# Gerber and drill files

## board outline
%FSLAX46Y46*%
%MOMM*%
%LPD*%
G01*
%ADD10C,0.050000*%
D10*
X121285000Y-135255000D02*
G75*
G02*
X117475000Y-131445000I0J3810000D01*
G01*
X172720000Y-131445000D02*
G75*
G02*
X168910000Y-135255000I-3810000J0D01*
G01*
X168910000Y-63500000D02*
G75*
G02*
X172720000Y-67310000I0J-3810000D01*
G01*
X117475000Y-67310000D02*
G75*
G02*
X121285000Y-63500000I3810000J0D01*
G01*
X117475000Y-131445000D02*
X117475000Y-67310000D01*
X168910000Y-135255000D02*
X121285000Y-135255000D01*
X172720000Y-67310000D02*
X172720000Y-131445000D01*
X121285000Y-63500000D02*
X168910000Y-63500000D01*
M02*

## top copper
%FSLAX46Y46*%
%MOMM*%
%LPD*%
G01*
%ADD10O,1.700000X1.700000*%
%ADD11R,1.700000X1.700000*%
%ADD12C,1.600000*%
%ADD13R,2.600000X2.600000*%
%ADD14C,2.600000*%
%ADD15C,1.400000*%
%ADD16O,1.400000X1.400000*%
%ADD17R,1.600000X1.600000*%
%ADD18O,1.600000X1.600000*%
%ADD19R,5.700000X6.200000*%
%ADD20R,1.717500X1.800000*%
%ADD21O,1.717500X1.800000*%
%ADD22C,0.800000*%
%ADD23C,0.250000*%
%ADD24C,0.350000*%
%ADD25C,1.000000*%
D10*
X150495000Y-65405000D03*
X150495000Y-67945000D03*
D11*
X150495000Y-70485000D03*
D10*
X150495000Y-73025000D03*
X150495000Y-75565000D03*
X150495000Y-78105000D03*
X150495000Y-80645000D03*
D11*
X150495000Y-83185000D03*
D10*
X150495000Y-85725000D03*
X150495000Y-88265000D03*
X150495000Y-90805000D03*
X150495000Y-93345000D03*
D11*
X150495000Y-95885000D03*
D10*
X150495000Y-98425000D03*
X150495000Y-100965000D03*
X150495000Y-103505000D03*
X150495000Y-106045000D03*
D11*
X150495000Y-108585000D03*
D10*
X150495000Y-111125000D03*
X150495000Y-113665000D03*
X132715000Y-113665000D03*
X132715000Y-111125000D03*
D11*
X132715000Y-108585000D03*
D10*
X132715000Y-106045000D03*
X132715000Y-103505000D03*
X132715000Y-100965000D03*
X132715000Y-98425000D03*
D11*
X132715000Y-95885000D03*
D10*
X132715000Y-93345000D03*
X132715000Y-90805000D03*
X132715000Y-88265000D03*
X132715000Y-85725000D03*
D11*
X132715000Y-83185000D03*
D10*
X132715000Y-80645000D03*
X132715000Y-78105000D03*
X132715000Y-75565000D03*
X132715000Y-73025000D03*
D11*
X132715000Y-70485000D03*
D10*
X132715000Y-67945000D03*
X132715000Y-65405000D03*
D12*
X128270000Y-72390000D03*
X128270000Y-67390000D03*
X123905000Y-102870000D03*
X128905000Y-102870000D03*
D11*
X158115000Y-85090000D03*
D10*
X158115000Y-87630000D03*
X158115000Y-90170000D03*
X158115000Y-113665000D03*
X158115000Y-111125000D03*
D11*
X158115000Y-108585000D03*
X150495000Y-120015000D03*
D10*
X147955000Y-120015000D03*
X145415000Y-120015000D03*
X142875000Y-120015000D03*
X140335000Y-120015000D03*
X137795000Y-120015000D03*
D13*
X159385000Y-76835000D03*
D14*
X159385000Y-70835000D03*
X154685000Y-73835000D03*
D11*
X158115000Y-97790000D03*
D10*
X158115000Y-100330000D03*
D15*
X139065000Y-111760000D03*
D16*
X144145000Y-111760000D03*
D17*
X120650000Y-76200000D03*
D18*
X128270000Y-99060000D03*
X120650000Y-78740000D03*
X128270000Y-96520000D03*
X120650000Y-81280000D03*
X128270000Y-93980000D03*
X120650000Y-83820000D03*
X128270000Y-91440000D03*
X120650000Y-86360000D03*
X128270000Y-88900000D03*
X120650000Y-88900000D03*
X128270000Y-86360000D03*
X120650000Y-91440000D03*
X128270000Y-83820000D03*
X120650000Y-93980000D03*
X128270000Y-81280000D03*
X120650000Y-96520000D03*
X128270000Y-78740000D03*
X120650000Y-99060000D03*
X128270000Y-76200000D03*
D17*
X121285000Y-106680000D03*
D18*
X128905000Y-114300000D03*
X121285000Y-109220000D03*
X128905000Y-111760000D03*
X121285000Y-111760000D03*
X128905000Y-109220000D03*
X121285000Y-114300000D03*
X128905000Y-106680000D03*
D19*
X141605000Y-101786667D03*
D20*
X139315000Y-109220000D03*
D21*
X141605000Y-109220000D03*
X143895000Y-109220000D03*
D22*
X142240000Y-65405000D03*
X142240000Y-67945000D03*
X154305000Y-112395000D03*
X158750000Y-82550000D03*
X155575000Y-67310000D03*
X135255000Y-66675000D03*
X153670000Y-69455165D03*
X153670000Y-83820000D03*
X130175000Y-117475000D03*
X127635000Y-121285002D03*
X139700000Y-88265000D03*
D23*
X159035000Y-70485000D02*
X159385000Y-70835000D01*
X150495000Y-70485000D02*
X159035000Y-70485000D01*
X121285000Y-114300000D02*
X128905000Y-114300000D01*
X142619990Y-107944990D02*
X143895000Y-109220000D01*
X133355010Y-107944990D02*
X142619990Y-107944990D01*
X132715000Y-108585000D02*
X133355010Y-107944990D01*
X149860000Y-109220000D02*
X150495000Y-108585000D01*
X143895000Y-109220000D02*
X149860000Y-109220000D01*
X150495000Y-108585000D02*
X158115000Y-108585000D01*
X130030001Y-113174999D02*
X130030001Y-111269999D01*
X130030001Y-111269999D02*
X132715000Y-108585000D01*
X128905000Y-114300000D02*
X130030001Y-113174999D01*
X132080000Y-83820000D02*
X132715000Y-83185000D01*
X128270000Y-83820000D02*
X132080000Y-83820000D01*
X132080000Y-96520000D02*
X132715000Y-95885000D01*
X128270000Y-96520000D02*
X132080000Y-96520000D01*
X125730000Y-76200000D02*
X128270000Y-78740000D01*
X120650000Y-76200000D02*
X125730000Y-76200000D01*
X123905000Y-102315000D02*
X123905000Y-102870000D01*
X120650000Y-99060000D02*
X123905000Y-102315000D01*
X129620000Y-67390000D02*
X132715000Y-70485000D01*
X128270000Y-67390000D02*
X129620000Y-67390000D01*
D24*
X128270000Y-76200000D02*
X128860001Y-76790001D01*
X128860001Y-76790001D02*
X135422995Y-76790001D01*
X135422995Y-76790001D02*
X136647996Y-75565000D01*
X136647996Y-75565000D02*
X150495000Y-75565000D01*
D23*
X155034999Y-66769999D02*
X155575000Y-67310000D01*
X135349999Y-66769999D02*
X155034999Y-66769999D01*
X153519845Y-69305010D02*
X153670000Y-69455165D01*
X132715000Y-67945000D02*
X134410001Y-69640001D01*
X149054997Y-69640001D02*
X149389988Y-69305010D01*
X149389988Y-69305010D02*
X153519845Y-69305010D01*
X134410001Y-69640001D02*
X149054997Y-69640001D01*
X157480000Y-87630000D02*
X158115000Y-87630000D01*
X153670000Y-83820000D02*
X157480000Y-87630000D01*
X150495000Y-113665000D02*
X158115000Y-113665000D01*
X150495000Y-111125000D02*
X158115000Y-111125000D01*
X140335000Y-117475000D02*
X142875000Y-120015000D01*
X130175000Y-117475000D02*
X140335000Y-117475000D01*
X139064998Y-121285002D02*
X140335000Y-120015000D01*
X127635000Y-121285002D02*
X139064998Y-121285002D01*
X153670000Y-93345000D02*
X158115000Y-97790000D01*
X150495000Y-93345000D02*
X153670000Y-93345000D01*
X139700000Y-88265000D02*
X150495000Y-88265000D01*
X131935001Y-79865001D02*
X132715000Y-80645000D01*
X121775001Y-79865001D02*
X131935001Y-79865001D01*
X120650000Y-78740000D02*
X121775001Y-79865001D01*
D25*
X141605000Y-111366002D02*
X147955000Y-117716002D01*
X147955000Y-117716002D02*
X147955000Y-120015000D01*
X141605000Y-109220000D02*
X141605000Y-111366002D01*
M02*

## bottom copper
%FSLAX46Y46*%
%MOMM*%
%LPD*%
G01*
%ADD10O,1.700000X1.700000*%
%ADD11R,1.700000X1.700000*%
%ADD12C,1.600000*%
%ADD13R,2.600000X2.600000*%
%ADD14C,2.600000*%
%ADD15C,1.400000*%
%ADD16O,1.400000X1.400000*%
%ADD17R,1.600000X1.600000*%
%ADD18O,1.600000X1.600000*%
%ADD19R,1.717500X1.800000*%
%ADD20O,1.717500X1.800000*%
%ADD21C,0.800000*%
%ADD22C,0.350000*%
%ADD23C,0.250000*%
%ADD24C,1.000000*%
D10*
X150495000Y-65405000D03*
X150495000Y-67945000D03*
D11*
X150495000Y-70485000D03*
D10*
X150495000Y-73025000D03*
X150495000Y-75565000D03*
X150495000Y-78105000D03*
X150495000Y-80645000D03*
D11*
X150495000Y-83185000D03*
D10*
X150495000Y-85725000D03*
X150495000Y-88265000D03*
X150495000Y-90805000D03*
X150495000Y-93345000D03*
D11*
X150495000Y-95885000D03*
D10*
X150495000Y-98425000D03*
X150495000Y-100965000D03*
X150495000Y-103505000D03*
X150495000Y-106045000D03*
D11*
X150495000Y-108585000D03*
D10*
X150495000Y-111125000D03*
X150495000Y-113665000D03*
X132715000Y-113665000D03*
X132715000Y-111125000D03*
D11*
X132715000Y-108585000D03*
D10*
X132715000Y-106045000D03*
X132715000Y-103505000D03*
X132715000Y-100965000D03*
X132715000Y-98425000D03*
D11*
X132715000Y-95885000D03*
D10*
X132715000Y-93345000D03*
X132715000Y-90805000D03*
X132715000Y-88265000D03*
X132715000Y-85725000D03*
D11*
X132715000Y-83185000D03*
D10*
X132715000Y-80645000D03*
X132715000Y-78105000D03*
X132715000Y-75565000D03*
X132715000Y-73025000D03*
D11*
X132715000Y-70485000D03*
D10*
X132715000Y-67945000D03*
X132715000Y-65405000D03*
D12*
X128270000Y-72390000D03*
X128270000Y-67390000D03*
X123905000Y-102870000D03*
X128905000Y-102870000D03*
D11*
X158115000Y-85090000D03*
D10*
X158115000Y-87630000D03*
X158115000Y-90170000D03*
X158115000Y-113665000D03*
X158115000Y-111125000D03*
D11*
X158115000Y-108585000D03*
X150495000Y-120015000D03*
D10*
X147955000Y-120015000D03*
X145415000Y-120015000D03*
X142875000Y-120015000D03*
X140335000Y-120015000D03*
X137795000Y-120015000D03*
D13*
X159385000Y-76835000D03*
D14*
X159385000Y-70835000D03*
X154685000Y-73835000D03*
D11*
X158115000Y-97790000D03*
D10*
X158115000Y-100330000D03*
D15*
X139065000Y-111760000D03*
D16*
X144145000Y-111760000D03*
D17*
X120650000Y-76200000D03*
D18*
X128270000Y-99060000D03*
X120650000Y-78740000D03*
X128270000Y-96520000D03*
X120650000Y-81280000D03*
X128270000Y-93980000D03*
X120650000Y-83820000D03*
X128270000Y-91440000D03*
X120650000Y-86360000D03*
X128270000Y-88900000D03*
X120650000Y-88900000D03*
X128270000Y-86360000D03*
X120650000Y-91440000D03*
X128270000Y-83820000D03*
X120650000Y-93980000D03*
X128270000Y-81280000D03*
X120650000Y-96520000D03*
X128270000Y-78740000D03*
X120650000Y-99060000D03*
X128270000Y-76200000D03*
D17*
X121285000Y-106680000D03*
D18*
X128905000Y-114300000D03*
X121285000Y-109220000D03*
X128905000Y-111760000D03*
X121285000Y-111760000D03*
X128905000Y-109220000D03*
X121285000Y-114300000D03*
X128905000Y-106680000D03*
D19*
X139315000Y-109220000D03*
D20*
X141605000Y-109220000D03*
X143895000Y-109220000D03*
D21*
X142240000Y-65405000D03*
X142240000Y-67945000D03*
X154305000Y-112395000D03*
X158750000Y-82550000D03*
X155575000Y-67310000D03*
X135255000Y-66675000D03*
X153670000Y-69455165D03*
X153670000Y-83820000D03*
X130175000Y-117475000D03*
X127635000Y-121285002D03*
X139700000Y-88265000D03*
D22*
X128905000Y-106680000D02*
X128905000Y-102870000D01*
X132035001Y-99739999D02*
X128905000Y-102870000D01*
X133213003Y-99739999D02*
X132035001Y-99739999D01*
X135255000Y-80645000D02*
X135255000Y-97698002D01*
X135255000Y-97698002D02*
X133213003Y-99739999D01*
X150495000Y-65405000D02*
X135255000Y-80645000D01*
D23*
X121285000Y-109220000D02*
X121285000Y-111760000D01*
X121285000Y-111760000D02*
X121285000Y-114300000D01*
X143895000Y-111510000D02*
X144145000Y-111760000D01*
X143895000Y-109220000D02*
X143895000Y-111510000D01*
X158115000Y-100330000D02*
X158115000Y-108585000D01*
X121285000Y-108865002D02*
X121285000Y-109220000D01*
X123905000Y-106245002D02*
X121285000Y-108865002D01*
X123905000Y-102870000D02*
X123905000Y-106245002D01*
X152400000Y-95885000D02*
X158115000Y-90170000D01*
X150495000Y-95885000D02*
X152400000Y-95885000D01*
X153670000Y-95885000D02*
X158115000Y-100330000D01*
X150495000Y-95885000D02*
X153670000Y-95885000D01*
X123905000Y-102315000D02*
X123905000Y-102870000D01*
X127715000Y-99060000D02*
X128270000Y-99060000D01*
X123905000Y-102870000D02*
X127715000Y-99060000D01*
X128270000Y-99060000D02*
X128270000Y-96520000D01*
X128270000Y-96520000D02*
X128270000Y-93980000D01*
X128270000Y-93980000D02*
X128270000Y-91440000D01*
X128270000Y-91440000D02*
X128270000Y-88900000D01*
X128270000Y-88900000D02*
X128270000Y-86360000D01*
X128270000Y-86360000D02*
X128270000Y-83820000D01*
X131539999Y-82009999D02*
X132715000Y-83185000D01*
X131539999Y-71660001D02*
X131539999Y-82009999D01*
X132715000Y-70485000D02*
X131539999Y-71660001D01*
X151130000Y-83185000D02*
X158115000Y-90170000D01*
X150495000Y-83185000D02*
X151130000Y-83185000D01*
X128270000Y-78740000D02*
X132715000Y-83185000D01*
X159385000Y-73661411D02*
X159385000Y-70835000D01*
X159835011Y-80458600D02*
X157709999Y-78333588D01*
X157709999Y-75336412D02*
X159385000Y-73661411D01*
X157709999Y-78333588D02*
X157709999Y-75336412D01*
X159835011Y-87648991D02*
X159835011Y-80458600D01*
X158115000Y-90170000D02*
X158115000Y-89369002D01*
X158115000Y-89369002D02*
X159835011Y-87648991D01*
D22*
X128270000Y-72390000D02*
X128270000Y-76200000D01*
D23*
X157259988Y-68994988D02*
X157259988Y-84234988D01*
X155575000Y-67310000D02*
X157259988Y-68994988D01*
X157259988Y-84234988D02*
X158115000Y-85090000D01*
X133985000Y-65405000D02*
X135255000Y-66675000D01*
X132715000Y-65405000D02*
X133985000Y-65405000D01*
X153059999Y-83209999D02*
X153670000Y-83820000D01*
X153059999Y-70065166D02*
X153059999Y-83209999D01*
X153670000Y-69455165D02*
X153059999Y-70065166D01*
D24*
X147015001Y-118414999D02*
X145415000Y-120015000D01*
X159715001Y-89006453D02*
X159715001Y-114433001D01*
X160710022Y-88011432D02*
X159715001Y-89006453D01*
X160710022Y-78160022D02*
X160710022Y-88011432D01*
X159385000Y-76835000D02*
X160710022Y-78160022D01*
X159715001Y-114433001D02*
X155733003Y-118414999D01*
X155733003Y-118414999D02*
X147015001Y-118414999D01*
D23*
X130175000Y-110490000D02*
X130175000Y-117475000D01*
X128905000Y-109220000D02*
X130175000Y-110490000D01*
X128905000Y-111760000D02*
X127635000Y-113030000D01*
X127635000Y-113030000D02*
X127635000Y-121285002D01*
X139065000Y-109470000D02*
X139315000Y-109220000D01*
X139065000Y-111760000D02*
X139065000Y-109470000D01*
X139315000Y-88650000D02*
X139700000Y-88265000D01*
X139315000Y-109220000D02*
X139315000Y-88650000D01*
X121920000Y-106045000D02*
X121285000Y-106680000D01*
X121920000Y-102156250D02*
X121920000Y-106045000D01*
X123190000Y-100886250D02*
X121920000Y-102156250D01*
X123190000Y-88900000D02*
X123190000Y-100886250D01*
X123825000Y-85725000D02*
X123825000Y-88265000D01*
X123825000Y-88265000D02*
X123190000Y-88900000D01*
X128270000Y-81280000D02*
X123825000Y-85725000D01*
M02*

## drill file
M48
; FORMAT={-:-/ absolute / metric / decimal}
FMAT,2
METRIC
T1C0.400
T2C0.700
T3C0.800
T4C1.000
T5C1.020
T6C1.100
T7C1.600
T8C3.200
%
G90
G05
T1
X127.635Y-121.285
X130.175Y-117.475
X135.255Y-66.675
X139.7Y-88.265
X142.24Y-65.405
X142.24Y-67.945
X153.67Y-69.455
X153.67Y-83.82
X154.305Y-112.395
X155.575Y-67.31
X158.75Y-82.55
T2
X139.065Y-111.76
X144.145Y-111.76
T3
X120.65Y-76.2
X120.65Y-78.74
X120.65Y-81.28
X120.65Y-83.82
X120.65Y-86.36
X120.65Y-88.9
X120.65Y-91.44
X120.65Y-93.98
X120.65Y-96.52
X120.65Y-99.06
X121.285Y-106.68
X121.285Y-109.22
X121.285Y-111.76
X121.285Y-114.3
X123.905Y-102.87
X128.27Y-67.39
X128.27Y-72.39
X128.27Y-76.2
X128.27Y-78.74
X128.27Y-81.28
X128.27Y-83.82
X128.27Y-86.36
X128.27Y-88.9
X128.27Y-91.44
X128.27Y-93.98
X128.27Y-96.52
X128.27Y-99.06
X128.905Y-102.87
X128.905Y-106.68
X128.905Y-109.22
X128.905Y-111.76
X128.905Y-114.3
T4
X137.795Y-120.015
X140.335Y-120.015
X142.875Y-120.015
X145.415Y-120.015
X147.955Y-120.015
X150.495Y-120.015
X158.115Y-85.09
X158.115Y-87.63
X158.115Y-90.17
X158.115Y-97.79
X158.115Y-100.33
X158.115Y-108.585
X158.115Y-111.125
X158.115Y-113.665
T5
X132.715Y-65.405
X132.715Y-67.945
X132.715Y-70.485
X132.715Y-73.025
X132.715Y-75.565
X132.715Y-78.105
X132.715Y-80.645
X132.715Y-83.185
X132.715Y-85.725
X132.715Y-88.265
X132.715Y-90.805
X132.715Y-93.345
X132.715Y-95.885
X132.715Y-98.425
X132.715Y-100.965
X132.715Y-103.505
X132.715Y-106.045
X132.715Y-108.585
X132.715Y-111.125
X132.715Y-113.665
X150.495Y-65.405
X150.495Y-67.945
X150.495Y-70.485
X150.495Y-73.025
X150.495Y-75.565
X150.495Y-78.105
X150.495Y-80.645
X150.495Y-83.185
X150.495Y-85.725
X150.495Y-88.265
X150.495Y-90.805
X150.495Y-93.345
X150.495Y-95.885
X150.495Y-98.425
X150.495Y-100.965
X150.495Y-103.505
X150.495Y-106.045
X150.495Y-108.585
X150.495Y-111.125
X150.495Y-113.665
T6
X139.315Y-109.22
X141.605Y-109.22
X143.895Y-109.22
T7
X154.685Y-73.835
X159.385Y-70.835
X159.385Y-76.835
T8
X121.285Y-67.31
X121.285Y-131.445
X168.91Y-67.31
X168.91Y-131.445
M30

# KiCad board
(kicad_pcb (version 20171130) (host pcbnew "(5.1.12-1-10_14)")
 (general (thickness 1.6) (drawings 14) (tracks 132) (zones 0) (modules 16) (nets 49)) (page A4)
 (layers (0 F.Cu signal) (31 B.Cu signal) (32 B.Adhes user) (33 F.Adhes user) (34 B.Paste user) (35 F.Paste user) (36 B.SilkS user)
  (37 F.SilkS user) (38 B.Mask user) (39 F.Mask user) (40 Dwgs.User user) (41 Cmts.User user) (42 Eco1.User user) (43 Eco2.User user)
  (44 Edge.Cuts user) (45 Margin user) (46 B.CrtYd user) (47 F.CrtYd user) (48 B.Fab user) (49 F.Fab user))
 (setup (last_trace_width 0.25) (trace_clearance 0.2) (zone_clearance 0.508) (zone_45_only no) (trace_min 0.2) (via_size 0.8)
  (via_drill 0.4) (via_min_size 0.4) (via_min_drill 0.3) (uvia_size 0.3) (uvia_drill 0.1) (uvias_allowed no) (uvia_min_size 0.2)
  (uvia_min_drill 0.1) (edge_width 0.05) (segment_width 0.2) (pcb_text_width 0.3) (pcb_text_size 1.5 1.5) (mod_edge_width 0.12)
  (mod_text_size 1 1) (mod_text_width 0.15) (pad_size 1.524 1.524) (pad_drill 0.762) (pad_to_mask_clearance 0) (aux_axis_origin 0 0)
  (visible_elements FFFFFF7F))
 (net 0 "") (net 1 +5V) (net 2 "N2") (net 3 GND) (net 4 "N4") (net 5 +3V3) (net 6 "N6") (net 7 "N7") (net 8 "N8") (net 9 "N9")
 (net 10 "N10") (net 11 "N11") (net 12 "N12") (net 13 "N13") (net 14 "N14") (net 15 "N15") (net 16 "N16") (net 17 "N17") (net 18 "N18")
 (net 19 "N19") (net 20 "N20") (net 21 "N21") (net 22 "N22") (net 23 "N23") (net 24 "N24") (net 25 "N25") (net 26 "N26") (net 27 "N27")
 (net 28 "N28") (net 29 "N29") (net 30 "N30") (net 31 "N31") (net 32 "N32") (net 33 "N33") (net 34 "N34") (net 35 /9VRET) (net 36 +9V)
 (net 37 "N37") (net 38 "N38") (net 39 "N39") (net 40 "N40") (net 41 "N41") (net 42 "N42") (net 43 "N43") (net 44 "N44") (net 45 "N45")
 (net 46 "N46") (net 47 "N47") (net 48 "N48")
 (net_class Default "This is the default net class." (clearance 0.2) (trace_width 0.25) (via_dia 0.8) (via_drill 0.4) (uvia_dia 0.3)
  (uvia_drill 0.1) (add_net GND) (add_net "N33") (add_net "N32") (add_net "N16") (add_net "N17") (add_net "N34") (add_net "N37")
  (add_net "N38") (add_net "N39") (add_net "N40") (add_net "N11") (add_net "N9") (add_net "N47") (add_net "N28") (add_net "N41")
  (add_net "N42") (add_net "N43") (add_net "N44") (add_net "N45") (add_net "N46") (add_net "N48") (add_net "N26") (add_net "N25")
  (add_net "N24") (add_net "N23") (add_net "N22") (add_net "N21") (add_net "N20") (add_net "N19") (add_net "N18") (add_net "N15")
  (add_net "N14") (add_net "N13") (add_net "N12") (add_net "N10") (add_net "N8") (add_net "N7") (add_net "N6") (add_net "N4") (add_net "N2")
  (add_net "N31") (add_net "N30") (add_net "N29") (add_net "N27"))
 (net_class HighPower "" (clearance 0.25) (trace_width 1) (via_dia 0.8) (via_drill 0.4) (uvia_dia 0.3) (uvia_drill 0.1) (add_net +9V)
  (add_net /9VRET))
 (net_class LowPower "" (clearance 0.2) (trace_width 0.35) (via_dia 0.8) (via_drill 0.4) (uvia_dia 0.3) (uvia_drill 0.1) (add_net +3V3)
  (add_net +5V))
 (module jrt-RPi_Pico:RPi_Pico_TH (layer F.Cu) (at 141.605 89.535)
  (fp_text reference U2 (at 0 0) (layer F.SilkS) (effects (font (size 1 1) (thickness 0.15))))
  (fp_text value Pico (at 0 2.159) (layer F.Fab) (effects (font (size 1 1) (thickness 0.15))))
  (pad 40 thru_hole oval (at 8.89 -24.13) (size 1.7 1.7) (drill 1.02) (layers *.Cu *.Mask) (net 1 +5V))
  (pad 39 thru_hole oval (at 8.89 -21.59) (size 1.7 1.7) (drill 1.02) (layers *.Cu *.Mask) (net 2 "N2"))
  (pad 38 thru_hole rect (at 8.89 -19.05) (size 1.7 1.7) (drill 1.02) (layers *.Cu *.Mask) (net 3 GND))
  (pad 37 thru_hole oval (at 8.89 -16.51) (size 1.7 1.7) (drill 1.02) (layers *.Cu *.Mask) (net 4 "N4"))
  (pad 36 thru_hole oval (at 8.89 -13.97) (size 1.7 1.7) (drill 1.02) (layers *.Cu *.Mask) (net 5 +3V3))
  (pad 35 thru_hole oval (at 8.89 -11.43) (size 1.7 1.7) (drill 1.02) (layers *.Cu *.Mask) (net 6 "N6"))
  (pad 34 thru_hole oval (at 8.89 -8.89) (size 1.7 1.7) (drill 1.02) (layers *.Cu *.Mask) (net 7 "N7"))
  (pad 33 thru_hole rect (at 8.89 -6.35) (size 1.7 1.7) (drill 1.02) (layers *.Cu *.Mask) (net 3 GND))
  (pad 32 thru_hole oval (at 8.89 -3.81) (size 1.7 1.7) (drill 1.02) (layers *.Cu *.Mask) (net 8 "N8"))
  (pad 31 thru_hole oval (at 8.89 -1.27) (size 1.7 1.7) (drill 1.02) (layers *.Cu *.Mask) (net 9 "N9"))
  (pad 30 thru_hole oval (at 8.89 1.27) (size 1.7 1.7) (drill 1.02) (layers *.Cu *.Mask) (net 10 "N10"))
  (pad 29 thru_hole oval (at 8.89 3.81) (size 1.7 1.7) (drill 1.02) (layers *.Cu *.Mask) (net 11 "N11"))
  (pad 28 thru_hole rect (at 8.89 6.35) (size 1.7 1.7) (drill 1.02) (layers *.Cu *.Mask) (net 3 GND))
  (pad 27 thru_hole oval (at 8.89 8.89) (size 1.7 1.7) (drill 1.02) (layers *.Cu *.Mask) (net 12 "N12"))
  (pad 26 thru_hole oval (at 8.89 11.43) (size 1.7 1.7) (drill 1.02) (layers *.Cu *.Mask) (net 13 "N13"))
  (pad 25 thru_hole oval (at 8.89 13.97) (size 1.7 1.7) (drill 1.02) (layers *.Cu *.Mask) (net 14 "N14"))
  (pad 24 thru_hole oval (at 8.89 16.51) (size 1.7 1.7) (drill 1.02) (layers *.Cu *.Mask) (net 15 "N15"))
  (pad 23 thru_hole rect (at 8.89 19.05) (size 1.7 1.7) (drill 1.02) (layers *.Cu *.Mask) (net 3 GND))
  (pad 22 thru_hole oval (at 8.89 21.59) (size 1.7 1.7) (drill 1.02) (layers *.Cu *.Mask) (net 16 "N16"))
  (pad 21 thru_hole oval (at 8.89 24.13) (size 1.7 1.7) (drill 1.02) (layers *.Cu *.Mask) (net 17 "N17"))
  (pad 20 thru_hole oval (at -8.89 24.13) (size 1.7 1.7) (drill 1.02) (layers *.Cu *.Mask) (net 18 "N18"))
  (pad 19 thru_hole oval (at -8.89 21.59) (size 1.7 1.7) (drill 1.02) (layers *.Cu *.Mask) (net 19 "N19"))
  (pad 18 thru_hole rect (at -8.89 19.05) (size 1.7 1.7) (drill 1.02) (layers *.Cu *.Mask) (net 3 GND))
  (pad 17 thru_hole oval (at -8.89 16.51) (size 1.7 1.7) (drill 1.02) (layers *.Cu *.Mask) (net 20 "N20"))
  (pad 16 thru_hole oval (at -8.89 13.97) (size 1.7 1.7) (drill 1.02) (layers *.Cu *.Mask) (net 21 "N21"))
  (pad 15 thru_hole oval (at -8.89 11.43) (size 1.7 1.7) (drill 1.02) (layers *.Cu *.Mask) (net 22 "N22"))
  (pad 14 thru_hole oval (at -8.89 8.89) (size 1.7 1.7) (drill 1.02) (layers *.Cu *.Mask) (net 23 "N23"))
  (pad 13 thru_hole rect (at -8.89 6.35) (size 1.7 1.7) (drill 1.02) (layers *.Cu *.Mask) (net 3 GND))
  (pad 12 thru_hole oval (at -8.89 3.81) (size 1.7 1.7) (drill 1.02) (layers *.Cu *.Mask) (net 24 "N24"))
  (pad 11 thru_hole oval (at -8.89 1.27) (size 1.7 1.7) (drill 1.02) (layers *.Cu *.Mask) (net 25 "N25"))
  (pad 10 thru_hole oval (at -8.89 -1.27) (size 1.7 1.7) (drill 1.02) (layers *.Cu *.Mask) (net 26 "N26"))
  (pad 9 thru_hole oval (at -8.89 -3.81) (size 1.7 1.7) (drill 1.02) (layers *.Cu *.Mask) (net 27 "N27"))
  (pad 8 thru_hole rect (at -8.89 -6.35) (size 1.7 1.7) (drill 1.02) (layers *.Cu *.Mask) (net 3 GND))
  (pad 7 thru_hole oval (at -8.89 -8.89) (size 1.7 1.7) (drill 1.02) (layers *.Cu *.Mask) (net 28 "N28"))
  (pad 6 thru_hole oval (at -8.89 -11.43) (size 1.7 1.7) (drill 1.02) (layers *.Cu *.Mask) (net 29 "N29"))
  (pad 5 thru_hole oval (at -8.89 -13.97) (size 1.7 1.7) (drill 1.02) (layers *.Cu *.Mask) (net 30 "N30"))
  (pad 4 thru_hole oval (at -8.89 -16.51) (size 1.7 1.7) (drill 1.02) (layers *.Cu *.Mask) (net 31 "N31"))
  (pad 3 thru_hole rect (at -8.89 -19.05) (size 1.7 1.7) (drill 1.02) (layers *.Cu *.Mask) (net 3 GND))
  (pad 2 thru_hole oval (at -8.89 -21.59) (size 1.7 1.7) (drill 1.02) (layers *.Cu *.Mask) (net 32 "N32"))
  (pad 1 thru_hole oval (at -8.89 -24.13) (size 1.7 1.7) (drill 1.02) (layers *.Cu *.Mask) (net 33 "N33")))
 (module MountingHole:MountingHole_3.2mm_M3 (layer F.Cu) (at 168.91 67.31)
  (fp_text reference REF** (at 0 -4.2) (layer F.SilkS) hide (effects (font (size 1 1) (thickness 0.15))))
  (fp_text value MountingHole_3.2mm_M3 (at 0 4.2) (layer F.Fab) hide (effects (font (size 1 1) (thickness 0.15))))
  (pad 1 np_thru_hole circle (at 0 0) (size 3.2 3.2) (drill 3.2) (layers *.Cu *.Mask)))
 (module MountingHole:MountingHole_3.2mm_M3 (layer F.Cu) (at 168.91 131.445)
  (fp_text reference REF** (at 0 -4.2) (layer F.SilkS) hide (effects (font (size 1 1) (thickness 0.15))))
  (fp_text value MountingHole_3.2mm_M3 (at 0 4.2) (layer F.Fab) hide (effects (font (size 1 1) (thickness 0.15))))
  (pad 1 np_thru_hole circle (at 0 0) (size 3.2 3.2) (drill 3.2) (layers *.Cu *.Mask)))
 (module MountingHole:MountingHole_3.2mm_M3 (layer F.Cu) (at 121.285 131.445)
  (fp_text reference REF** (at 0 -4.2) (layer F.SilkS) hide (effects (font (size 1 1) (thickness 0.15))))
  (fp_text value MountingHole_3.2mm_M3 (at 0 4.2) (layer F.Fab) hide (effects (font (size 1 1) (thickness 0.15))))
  (pad 1 np_thru_hole circle (at 0 0) (size 3.2 3.2) (drill 3.2) (layers *.Cu *.Mask)))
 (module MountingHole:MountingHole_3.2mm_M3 (layer F.Cu) (at 121.285 67.31)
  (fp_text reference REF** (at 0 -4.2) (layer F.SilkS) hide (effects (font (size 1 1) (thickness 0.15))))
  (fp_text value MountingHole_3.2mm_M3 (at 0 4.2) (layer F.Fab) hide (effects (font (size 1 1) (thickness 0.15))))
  (pad 1 np_thru_hole circle (at 0 0) (size 3.2 3.2) (drill 3.2) (layers *.Cu *.Mask)))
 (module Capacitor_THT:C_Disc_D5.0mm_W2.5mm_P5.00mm (layer F.Cu) (at 128.27 72.39 90)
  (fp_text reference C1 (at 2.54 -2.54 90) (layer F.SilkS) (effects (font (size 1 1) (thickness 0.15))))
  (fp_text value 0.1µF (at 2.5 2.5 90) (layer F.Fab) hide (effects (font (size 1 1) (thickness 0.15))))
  (pad 1 thru_hole circle (at 0 0 90) (size 1.6 1.6) (drill 0.8) (layers *.Cu *.Mask) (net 5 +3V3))
  (pad 2 thru_hole circle (at 5 0 90) (size 1.6 1.6) (drill 0.8) (layers *.Cu *.Mask) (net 3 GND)))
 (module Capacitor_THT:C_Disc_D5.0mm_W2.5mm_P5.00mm (layer F.Cu) (at 128.905 102.87 180)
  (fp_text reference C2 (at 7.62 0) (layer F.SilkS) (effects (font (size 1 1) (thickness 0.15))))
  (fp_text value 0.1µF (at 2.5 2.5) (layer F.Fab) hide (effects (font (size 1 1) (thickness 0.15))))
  (pad 2 thru_hole circle (at 5 0 180) (size 1.6 1.6) (drill 0.8) (layers *.Cu *.Mask) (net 3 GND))
  (pad 1 thru_hole circle (at 0 0 180) (size 1.6 1.6) (drill 0.8) (layers *.Cu *.Mask) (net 1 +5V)))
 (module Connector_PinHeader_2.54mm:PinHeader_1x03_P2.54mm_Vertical (layer F.Cu) (at 158.115 85.09)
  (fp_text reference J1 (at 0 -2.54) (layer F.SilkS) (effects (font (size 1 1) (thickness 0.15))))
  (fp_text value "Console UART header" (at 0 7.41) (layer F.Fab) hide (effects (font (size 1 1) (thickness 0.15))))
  (pad 1 thru_hole rect (at 0 0) (size 1.7 1.7) (drill 1) (layers *.Cu *.Mask) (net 33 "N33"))
  (pad 2 thru_hole oval (at 0 2.54) (size 1.7 1.7) (drill 1) (layers *.Cu *.Mask) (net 32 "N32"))
  (pad 3 thru_hole oval (at 0 5.08) (size 1.7 1.7) (drill 1) (layers *.Cu *.Mask) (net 3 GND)))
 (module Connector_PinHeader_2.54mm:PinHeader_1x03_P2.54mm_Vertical (layer F.Cu) (at 158.115 108.585)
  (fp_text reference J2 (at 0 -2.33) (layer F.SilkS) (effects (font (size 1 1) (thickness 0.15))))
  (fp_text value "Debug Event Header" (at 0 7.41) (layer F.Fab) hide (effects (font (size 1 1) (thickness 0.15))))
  (pad 3 thru_hole oval (at 0 5.08) (size 1.7 1.7) (drill 1) (layers *.Cu *.Mask) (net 17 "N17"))
  (pad 2 thru_hole oval (at 0 2.54) (size 1.7 1.7) (drill 1) (layers *.Cu *.Mask) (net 16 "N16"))
  (pad 1 thru_hole rect (at 0 0) (size 1.7 1.7) (drill 1) (layers *.Cu *.Mask) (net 3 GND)))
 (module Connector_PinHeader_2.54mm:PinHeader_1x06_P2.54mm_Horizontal (layer F.Cu) (at 150.495 120.015 270)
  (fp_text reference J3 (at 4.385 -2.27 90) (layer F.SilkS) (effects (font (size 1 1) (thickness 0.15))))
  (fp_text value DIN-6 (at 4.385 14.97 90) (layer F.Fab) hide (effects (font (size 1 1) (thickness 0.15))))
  (pad 1 thru_hole rect (at 0 0 270) (size 1.7 1.7) (drill 1) (layers *.Cu *.Mask) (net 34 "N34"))
  (pad 2 thru_hole oval (at 0 2.54 270) (size 1.7 1.7) (drill 1) (layers *.Cu *.Mask) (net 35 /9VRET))
  (pad 3 thru_hole oval (at 0 5.08 270) (size 1.7 1.7) (drill 1) (layers *.Cu *.Mask) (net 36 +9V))
  (pad 4 thru_hole oval (at 0 7.62 270) (size 1.7 1.7) (drill 1) (layers *.Cu *.Mask) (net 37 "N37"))
  (pad 5 thru_hole oval (at 0 10.16 270) (size 1.7 1.7) (drill 1) (layers *.Cu *.Mask) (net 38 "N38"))
  (pad 6 thru_hole oval (at 0 12.7 270) (size 1.7 1.7) (drill 1) (layers *.Cu *.Mask) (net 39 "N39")))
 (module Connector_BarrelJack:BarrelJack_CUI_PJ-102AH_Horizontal (layer F.Cu) (at 159.385 76.835 180)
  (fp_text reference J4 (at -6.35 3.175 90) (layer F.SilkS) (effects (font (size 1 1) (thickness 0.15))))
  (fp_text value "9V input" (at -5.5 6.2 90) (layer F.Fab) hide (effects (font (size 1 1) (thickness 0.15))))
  (pad 1 thru_hole rect (at 0 0 180) (size 2.6 2.6) (drill 1.6) (layers *.Cu *.Mask) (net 36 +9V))
  (pad 2 thru_hole circle (at 0 6 180) (size 2.6 2.6) (drill 1.6) (layers *.Cu *.Mask) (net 3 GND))
  (pad 3 thru_hole circle (at 4.7 3 180) (size 2.6 2.6) (drill 1.6) (layers *.Cu *.Mask) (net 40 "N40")))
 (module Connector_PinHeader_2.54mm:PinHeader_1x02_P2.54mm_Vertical (layer F.Cu) (at 158.115 97.79)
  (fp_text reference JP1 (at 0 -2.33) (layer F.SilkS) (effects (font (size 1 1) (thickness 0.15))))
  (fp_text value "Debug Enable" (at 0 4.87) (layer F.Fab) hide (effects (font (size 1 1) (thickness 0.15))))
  (pad 1 thru_hole rect (at 0 0) (size 1.7 1.7) (drill 1) (layers *.Cu *.Mask) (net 11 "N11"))
  (pad 2 thru_hole oval (at 0 2.54) (size 1.7 1.7) (drill 1) (layers *.Cu *.Mask) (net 3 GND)))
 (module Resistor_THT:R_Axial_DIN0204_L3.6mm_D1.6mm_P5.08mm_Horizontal (layer F.Cu) (at 139.065 111.76)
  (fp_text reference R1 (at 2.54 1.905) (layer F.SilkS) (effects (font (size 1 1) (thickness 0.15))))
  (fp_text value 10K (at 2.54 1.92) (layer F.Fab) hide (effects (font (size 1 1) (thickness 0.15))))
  (pad 1 thru_hole circle (at 0 0) (size 1.4 1.4) (drill 0.7) (layers *.Cu *.Mask) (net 9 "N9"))
  (pad 2 thru_hole oval (at 5.08 0) (size 1.4 1.4) (drill 0.7) (layers *.Cu *.Mask) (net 3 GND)))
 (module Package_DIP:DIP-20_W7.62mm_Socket (layer F.Cu) (at 120.65 76.2)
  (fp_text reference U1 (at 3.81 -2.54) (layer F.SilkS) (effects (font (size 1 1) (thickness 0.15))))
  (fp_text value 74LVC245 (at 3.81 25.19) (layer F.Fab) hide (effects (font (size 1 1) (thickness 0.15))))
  (pad 1 thru_hole rect (at 0 0) (size 1.6 1.6) (drill 0.8) (layers *.Cu *.Mask) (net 3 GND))
  (pad 11 thru_hole oval (at 7.62 22.86) (size 1.6 1.6) (drill 0.8) (layers *.Cu *.Mask) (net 3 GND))
  (pad 2 thru_hole oval (at 0 2.54) (size 1.6 1.6) (drill 0.8) (layers *.Cu *.Mask) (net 28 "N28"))
  (pad 12 thru_hole oval (at 7.62 20.32) (size 1.6 1.6) (drill 0.8) (layers *.Cu *.Mask) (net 3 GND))
  (pad 3 thru_hole oval (at 0 5.08) (size 1.6 1.6) (drill 0.8) (layers *.Cu *.Mask) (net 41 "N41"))
  (pad 13 thru_hole oval (at 7.62 17.78) (size 1.6 1.6) (drill 0.8) (layers *.Cu *.Mask) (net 3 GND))
  (pad 4 thru_hole oval (at 0 7.62) (size 1.6 1.6) (drill 0.8) (layers *.Cu *.Mask) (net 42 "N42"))
  (pad 14 thru_hole oval (at 7.62 15.24) (size 1.6 1.6) (drill 0.8) (layers *.Cu *.Mask) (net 3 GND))
  (pad 5 thru_hole oval (at 0 10.16) (size 1.6 1.6) (drill 0.8) (layers *.Cu *.Mask) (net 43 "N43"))
  (pad 15 thru_hole oval (at 7.62 12.7) (size 1.6 1.6) (drill 0.8) (layers *.Cu *.Mask) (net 3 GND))
  (pad 6 thru_hole oval (at 0 12.7) (size 1.6 1.6) (drill 0.8) (layers *.Cu *.Mask) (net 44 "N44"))
  (pad 16 thru_hole oval (at 7.62 10.16) (size 1.6 1.6) (drill 0.8) (layers *.Cu *.Mask) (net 3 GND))
  (pad 7 thru_hole oval (at 0 15.24) (size 1.6 1.6) (drill 0.8) (layers *.Cu *.Mask) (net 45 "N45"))
  (pad 17 thru_hole oval (at 7.62 7.62) (size 1.6 1.6) (drill 0.8) (layers *.Cu *.Mask) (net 3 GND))
  (pad 8 thru_hole oval (at 0 17.78) (size 1.6 1.6) (drill 0.8) (layers *.Cu *.Mask) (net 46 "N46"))
  (pad 18 thru_hole oval (at 7.62 5.08) (size 1.6 1.6) (drill 0.8) (layers *.Cu *.Mask) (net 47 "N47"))
  (pad 9 thru_hole oval (at 0 20.32) (size 1.6 1.6) (drill 0.8) (layers *.Cu *.Mask) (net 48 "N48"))
  (pad 19 thru_hole oval (at 7.62 2.54) (size 1.6 1.6) (drill 0.8) (layers *.Cu *.Mask) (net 3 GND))
  (pad 10 thru_hole oval (at 0 22.86) (size 1.6 1.6) (drill 0.8) (layers *.Cu *.Mask) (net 3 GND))
  (pad 20 thru_hole oval (at 7.62 0) (size 1.6 1.6) (drill 0.8) (layers *.Cu *.Mask) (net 5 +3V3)))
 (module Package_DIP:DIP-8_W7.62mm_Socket (layer F.Cu) (at 121.285 106.68)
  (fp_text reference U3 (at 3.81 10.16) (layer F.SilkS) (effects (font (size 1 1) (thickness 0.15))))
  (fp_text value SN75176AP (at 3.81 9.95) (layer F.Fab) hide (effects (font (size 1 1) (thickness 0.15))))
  (pad 1 thru_hole rect (at 0 0) (size 1.6 1.6) (drill 0.8) (layers *.Cu *.Mask) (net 47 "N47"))
  (pad 5 thru_hole oval (at 7.62 7.62) (size 1.6 1.6) (drill 0.8) (layers *.Cu *.Mask) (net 3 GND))
  (pad 2 thru_hole oval (at 0 2.54) (size 1.6 1.6) (drill 0.8) (layers *.Cu *.Mask) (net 3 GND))
  (pad 6 thru_hole oval (at 7.62 5.08) (size 1.6 1.6) (drill 0.8) (layers *.Cu *.Mask) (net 38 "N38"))
  (pad 3 thru_hole oval (at 0 5.08) (size 1.6 1.6) (drill 0.8) (layers *.Cu *.Mask) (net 3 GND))
  (pad 7 thru_hole oval (at 7.62 2.54) (size 1.6 1.6) (drill 0.8) (layers *.Cu *.Mask) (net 37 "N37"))
  (pad 4 thru_hole oval (at 0 7.62) (size 1.6 1.6) (drill 0.8) (layers *.Cu *.Mask) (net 3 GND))
  (pad 8 thru_hole oval (at 7.62 0) (size 1.6 1.6) (drill 0.8) (layers *.Cu *.Mask) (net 1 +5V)))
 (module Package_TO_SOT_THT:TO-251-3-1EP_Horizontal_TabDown (layer F.Cu) (at 139.315 109.22)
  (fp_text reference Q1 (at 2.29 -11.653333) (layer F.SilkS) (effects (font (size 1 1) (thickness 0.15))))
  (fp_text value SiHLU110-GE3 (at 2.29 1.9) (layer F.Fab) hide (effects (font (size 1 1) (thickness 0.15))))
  (pad 4 smd rect (at 2.29 -7.433333) (size 5.7 6.2) (layers F.Cu F.Paste F.Mask))
  (pad 1 thru_hole rect (at 0 0) (size 1.7175 1.8) (drill 1.1) (layers *.Cu *.Mask) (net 9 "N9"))
  (pad 2 thru_hole oval (at 2.29 0) (size 1.7175 1.8) (drill 1.1) (layers *.Cu *.Mask) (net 35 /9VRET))
  (pad 3 thru_hole oval (at 4.58 0) (size 1.7175 1.8) (drill 1.1) (layers *.Cu *.Mask) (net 3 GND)))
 (gr_arc (start 121.285 131.445) (end 117.475 131.445) (angle -90) (layer Edge.Cuts) (width 0.05))
 (gr_arc (start 168.91 131.445) (end 168.91 135.255) (angle -90) (layer Edge.Cuts) (width 0.05))
 (gr_arc (start 168.91 67.31) (end 172.72 67.31) (angle -90) (layer Edge.Cuts) (width 0.05))
 (gr_arc (start 121.285 67.31) (end 121.285 63.5) (angle -90) (layer Edge.Cuts) (width 0.05))
 (gr_line (start 117.475 131.445) (end 117.475 67.31) (layer Edge.Cuts) (width 0.05))
 (gr_line (start 168.91 135.255) (end 121.285 135.255) (layer Edge.Cuts) (width 0.05))
 (gr_line (start 172.72 67.31) (end 172.72 131.445) (layer Edge.Cuts) (width 0.05))
 (gr_line (start 121.285 63.5) (end 168.91 63.5) (layer Edge.Cuts) (width 0.05))
 (segment (start 128.905 106.68) (end 128.905 102.87) (width 0.35) (layer B.Cu) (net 1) (status 30))
 (segment (start 132.035001 99.739999) (end 128.905 102.87) (width 0.35) (layer B.Cu) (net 1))
 (segment (start 133.213003 99.739999) (end 132.035001 99.739999) (width 0.35) (layer B.Cu) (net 1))
 (segment (start 135.255 80.645) (end 135.255 97.698002) (width 0.35) (layer B.Cu) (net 1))
 (segment (start 135.255 97.698002) (end 133.213003 99.739999) (width 0.35) (layer B.Cu) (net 1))
 (segment (start 150.495 65.405) (end 135.255 80.645) (width 0.35) (layer B.Cu) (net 1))
 (segment (start 159.035 70.485) (end 159.385 70.835) (width 0.25) (layer F.Cu) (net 3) (status 30))
 (segment (start 150.495 70.485) (end 159.035 70.485) (width 0.25) (layer F.Cu) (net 3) (status 30))
 (segment (start 121.285 109.22) (end 121.285 111.76) (width 0.25) (layer B.Cu) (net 3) (status 30))
 (segment (start 121.285 111.76) (end 121.285 114.3) (width 0.25) (layer B.Cu) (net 3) (status 30))
 (segment (start 121.285 114.3) (end 128.905 114.3) (width 0.25) (layer F.Cu) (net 3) (status 30))
 (segment (start 142.61999 107.94499) (end 143.895 109.22) (width 0.25) (layer F.Cu) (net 3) (status 20))
 (segment (start 133.35501 107.94499) (end 142.61999 107.94499) (width 0.25) (layer F.Cu) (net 3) (status 10))
 (segment (start 132.715 108.585) (end 133.35501 107.94499) (width 0.25) (layer F.Cu) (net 3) (status 30))
 (segment (start 143.895 111.51) (end 144.145 111.76) (width 0.25) (layer B.Cu) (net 3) (status 30))
 (segment (start 143.895 109.22) (end 143.895 111.51) (width 0.25) (layer B.Cu) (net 3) (status 30))
 (segment (start 149.86 109.22) (end 150.495 108.585) (width 0.25) (layer F.Cu) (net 3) (status 30))
 (segment (start 143.895 109.22) (end 149.86 109.22) (width 0.25) (layer F.Cu) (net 3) (status 30))
 (segment (start 150.495 108.585) (end 158.115 108.585) (width 0.25) (layer F.Cu) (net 3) (status 30))
 (segment (start 158.115 100.33) (end 158.115 108.585) (width 0.25) (layer B.Cu) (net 3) (status 30))
 (segment (start 121.285 108.865002) (end 121.285 109.22) (width 0.25) (layer B.Cu) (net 3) (status 30))
 (segment (start 123.905 106.245002) (end 121.285 108.865002) (width 0.25) (layer B.Cu) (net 3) (status 20))
 (segment (start 123.905 102.87) (end 123.905 106.245002) (width 0.25) (layer B.Cu) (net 3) (status 10))
 (segment (start 130.030001 113.174999) (end 130.030001 111.269999) (width 0.25) (layer F.Cu) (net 3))
 (segment (start 130.030001 111.269999) (end 132.715 108.585) (width 0.25) (layer F.Cu) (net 3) (status 20))
 (segment (start 128.905 114.3) (end 130.030001 113.174999) (width 0.25) (layer F.Cu) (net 3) (status 10))
 (segment (start 152.4 95.885) (end 158.115 90.17) (width 0.25) (layer B.Cu) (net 3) (status 20))
 (segment (start 150.495 95.885) (end 152.4 95.885) (width 0.25) (layer B.Cu) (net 3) (status 10))
 (segment (start 153.67 95.885) (end 158.115 100.33) (width 0.25) (layer B.Cu) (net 3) (status 20))
 (segment (start 150.495 95.885) (end 153.67 95.885) (width 0.25) (layer B.Cu) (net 3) (status 10))
 (segment (start 123.905 102.315) (end 123.905 102.87) (width 0.25) (layer B.Cu) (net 3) (status 30))
 (segment (start 127.715 99.06) (end 128.27 99.06) (width 0.25) (layer B.Cu) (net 3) (status 30))
 (segment (start 123.905 102.87) (end 127.715 99.06) (width 0.25) (layer B.Cu) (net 3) (status 30))
 (segment (start 128.27 99.06) (end 128.27 96.52) (width 0.25) (layer B.Cu) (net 3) (status 30))
 (segment (start 128.27 96.52) (end 128.27 93.98) (width 0.25) (layer B.Cu) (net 3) (status 30))
 (segment (start 128.27 93.98) (end 128.27 91.44) (width 0.25) (layer B.Cu) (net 3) (status 30))
 (segment (start 128.27 91.44) (end 128.27 88.9) (width 0.25) (layer B.Cu) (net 3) (status 30))
 (segment (start 128.27 88.9) (end 128.27 86.36) (width 0.25) (layer B.Cu) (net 3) (status 30))
 (segment (start 128.27 86.36) (end 128.27 83.82) (width 0.25) (layer B.Cu) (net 3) (status 30))
 (segment (start 132.08 83.82) (end 132.715 83.185) (width 0.25) (layer F.Cu) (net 3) (status 30))
 (segment (start 128.27 83.82) (end 132.08 83.82) (width 0.25) (layer F.Cu) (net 3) (status 30))
 (segment (start 132.08 96.52) (end 132.715 95.885) (width 0.25) (layer F.Cu) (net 3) (status 30))
 (segment (start 128.27 96.52) (end 132.08 96.52) (width 0.25) (layer F.Cu) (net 3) (status 30))
 (segment (start 125.73 76.2) (end 128.27 78.74) (width 0.25) (layer F.Cu) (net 3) (status 20))
 (segment (start 120.65 76.2) (end 125.73 76.2) (width 0.25) (layer F.Cu) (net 3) (status 10))
 (segment (start 123.905 102.315) (end 123.905 102.87) (width 0.25) (layer F.Cu) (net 3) (status 30))
 (segment (start 120.65 99.06) (end 123.905 102.315) (width 0.25) (layer F.Cu) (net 3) (status 30))
 (segment (start 129.62 67.39) (end 132.715 70.485) (width 0.25) (layer F.Cu) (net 3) (status 20))
 (segment (start 128.27 67.39) (end 129.62 67.39) (width 0.25) (layer F.Cu) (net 3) (status 10))
 (segment (start 131.539999 82.009999) (end 132.715 83.185) (width 0.25) (layer B.Cu) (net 3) (status 20))
 (segment (start 131.539999 71.660001) (end 131.539999 82.009999) (width 0.25) (layer B.Cu) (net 3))
 (segment (start 132.715 70.485) (end 131.539999 71.660001) (width 0.25) (layer B.Cu) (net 3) (status 10))
 (segment (start 151.13 83.185) (end 158.115 90.17) (width 0.25) (layer B.Cu) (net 3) (status 30))
 (segment (start 150.495 83.185) (end 151.13 83.185) (width 0.25) (layer B.Cu) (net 3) (status 30))
 (segment (start 128.27 78.74) (end 132.715 83.185) (width 0.25) (layer B.Cu) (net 3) (status 30))
 (segment (start 159.385 73.661411) (end 159.385 70.835) (width 0.25) (layer B.Cu) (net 3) (status 20))
 (segment (start 159.835011 80.4586) (end 157.709999 78.333588) (width 0.25) (layer B.Cu) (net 3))
 (segment (start 157.709999 75.336412) (end 159.385 73.661411) (width 0.25) (layer B.Cu) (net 3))
 (segment (start 157.709999 78.333588) (end 157.709999 75.336412) (width 0.25) (layer B.Cu) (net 3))
 (segment (start 159.835011 87.648991) (end 159.835011 80.4586) (width 0.25) (layer B.Cu) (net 3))
 (segment (start 158.115 90.17) (end 158.115 89.369002) (width 0.25) (layer B.Cu) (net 3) (status 30))
 (segment (start 158.115 89.369002) (end 159.835011 87.648991) (width 0.25) (layer B.Cu) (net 3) (status 10))
 (via (at 142.24 65.405) (size 0.8) (drill 0.4) (layers F.Cu B.Cu) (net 3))
 (via (at 142.24 67.945) (size 0.8) (drill 0.4) (layers F.Cu B.Cu) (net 3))
 (via (at 154.305 112.395) (size 0.8) (drill 0.4) (layers F.Cu B.Cu) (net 3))
 (via (at 158.75 82.55) (size 0.8) (drill 0.4) (layers F.Cu B.Cu) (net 3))
 (segment (start 128.27 72.39) (end 128.27 76.2) (width 0.35) (layer B.Cu) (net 5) (status 30))
 (segment (start 128.27 76.2) (end 128.860001 76.790001) (width 0.35) (layer F.Cu) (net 5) (status 10))
 (segment (start 128.860001 76.790001) (end 135.422995 76.790001) (width 0.35) (layer F.Cu) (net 5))
 (segment (start 135.422995 76.790001) (end 136.647996 75.565) (width 0.35) (layer F.Cu) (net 5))
 (segment (start 136.647996 75.565) (end 150.495 75.565) (width 0.35) (layer F.Cu) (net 5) (status 20))
 (via (at 155.575 67.31) (size 0.8) (drill 0.4) (layers F.Cu B.Cu) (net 33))
 (segment (start 155.034999 66.769999) (end 155.575 67.31) (width 0.25) (layer F.Cu) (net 33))
 (segment (start 135.349999 66.769999) (end 155.034999 66.769999) (width 0.25) (layer F.Cu) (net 33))
 (segment (start 157.259988 68.994988) (end 157.259988 84.234988) (width 0.25) (layer B.Cu) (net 33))
 (segment (start 155.575 67.31) (end 157.259988 68.994988) (width 0.25) (layer B.Cu) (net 33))
 (segment (start 157.259988 84.234988) (end 158.115 85.09) (width 0.25) (layer B.Cu) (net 33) (status 20))
 (segment (start 133.985 65.405) (end 135.255 66.675) (width 0.25) (layer B.Cu) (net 33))
 (via (at 135.255 66.675) (size 0.8) (drill 0.4) (layers F.Cu B.Cu) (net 33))
 (segment (start 132.715 65.405) (end 133.985 65.405) (width 0.25) (layer B.Cu) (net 33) (status 10))
 (segment (start 153.519845 69.30501) (end 153.67 69.455165) (width 0.25) (layer F.Cu) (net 32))
 (segment (start 132.715 67.945) (end 134.410001 69.640001) (width 0.25) (layer F.Cu) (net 32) (status 10))
 (segment (start 149.054997 69.640001) (end 149.389988 69.30501) (width 0.25) (layer F.Cu) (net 32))
 (segment (start 149.389988 69.30501) (end 153.519845 69.30501) (width 0.25) (layer F.Cu) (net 32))
 (segment (start 134.410001 69.640001) (end 149.054997 69.640001) (width 0.25) (layer F.Cu) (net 32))
 (via (at 153.67 69.455165) (size 0.8) (drill 0.4) (layers F.Cu B.Cu) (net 32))
 (via (at 153.67 83.82) (size 0.8) (drill 0.4) (layers F.Cu B.Cu) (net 32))
 (segment (start 153.059999 83.209999) (end 153.67 83.82) (width 0.25) (layer B.Cu) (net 32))
 (segment (start 153.059999 70.065166) (end 153.059999 83.209999) (width 0.25) (layer B.Cu) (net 32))
 (segment (start 153.67 69.455165) (end 153.059999 70.065166) (width 0.25) (layer B.Cu) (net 32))
 (segment (start 157.48 87.63) (end 158.115 87.63) (width 0.25) (layer F.Cu) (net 32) (status 30))
 (segment (start 153.67 83.82) (end 157.48 87.63) (width 0.25) (layer F.Cu) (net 32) (status 20))
 (segment (start 150.495 113.665) (end 158.115 113.665) (width 0.25) (layer F.Cu) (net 17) (status 30))
 (segment (start 150.495 111.125) (end 158.115 111.125) (width 0.25) (layer F.Cu) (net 16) (status 30))
 (segment (start 147.015001 118.414999) (end 145.415 120.015) (width 1) (layer B.Cu) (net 36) (status 20))
 (segment (start 159.715001 89.006453) (end 159.715001 114.433001) (width 1) (layer B.Cu) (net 36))
 (segment (start 160.710022 88.011432) (end 159.715001 89.006453) (width 1) (layer B.Cu) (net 36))
 (segment (start 160.710022 78.160022) (end 160.710022 88.011432) (width 1) (layer B.Cu) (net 36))
 (segment (start 159.385 76.835) (end 160.710022 78.160022) (width 1) (layer B.Cu) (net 36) (status 10))
 (segment (start 159.715001 114.433001) (end 155.733003 118.414999) (width 1) (layer B.Cu) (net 36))
 (segment (start 155.733003 118.414999) (end 147.015001 118.414999) (width 1) (layer B.Cu) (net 36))
 (via (at 130.175 117.475) (size 0.8) (drill 0.4) (layers F.Cu B.Cu) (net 37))
 (segment (start 130.175 110.49) (end 130.175 117.475) (width 0.25) (layer B.Cu) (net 37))
 (segment (start 128.905 109.22) (end 130.175 110.49) (width 0.25) (layer B.Cu) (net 37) (status 10))
 (segment (start 140.335 117.475) (end 142.875 120.015) (width 0.25) (layer F.Cu) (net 37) (status 20))
 (segment (start 130.175 117.475) (end 140.335 117.475) (width 0.25) (layer F.Cu) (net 37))
 (via (at 127.635 121.285002) (size 0.8) (drill 0.4) (layers F.Cu B.Cu) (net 38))
 (segment (start 128.905 111.76) (end 127.635 113.03) (width 0.25) (layer B.Cu) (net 38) (status 10))
 (segment (start 127.635 113.03) (end 127.635 121.285002) (width 0.25) (layer B.Cu) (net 38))
 (segment (start 139.064998 121.285002) (end 140.335 120.015) (width 0.25) (layer F.Cu) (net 38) (status 20))
 (segment (start 127.635 121.285002) (end 139.064998 121.285002) (width 0.25) (layer F.Cu) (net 38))
 (segment (start 153.67 93.345) (end 158.115 97.79) (width 0.25) (layer F.Cu) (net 11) (status 20))
 (segment (start 150.495 93.345) (end 153.67 93.345) (width 0.25) (layer F.Cu) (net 11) (status 10))
 (segment (start 139.065 109.47) (end 139.315 109.22) (width 0.25) (layer B.Cu) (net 9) (status 30))
 (segment (start 139.065 111.76) (end 139.065 109.47) (width 0.25) (layer B.Cu) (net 9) (status 30))
 (via (at 139.7 88.265) (size 0.8) (drill 0.4) (layers F.Cu B.Cu) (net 9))
 (segment (start 139.315 88.65) (end 139.7 88.265) (width 0.25) (layer B.Cu) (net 9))
 (segment (start 139.315 109.22) (end 139.315 88.65) (width 0.25) (layer B.Cu) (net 9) (status 10))
 (segment (start 139.7 88.265) (end 150.495 88.265) (width 0.25) (layer F.Cu) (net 9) (status 20))
 (segment (start 131.935001 79.865001) (end 132.715 80.645) (width 0.25) (layer F.Cu) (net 28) (status 20))
 (segment (start 121.775001 79.865001) (end 131.935001 79.865001) (width 0.25) (layer F.Cu) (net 28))
 (segment (start 120.65 78.74) (end 121.775001 79.865001) (width 0.25) (layer F.Cu) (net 28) (status 10))
 (segment (start 121.92 106.045) (end 121.285 106.68) (width 0.25) (layer B.Cu) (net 47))
 (segment (start 121.92 102.15625) (end 121.92 106.045) (width 0.25) (layer B.Cu) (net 47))
 (segment (start 123.19 100.88625) (end 121.92 102.15625) (width 0.25) (layer B.Cu) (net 47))
 (segment (start 123.19 88.9) (end 123.19 100.88625) (width 0.25) (layer B.Cu) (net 47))
 (segment (start 123.825 85.725) (end 123.825 88.265) (width 0.25) (layer B.Cu) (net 47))
 (segment (start 123.825 88.265) (end 123.19 88.9) (width 0.25) (layer B.Cu) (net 47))
 (segment (start 128.27 81.28) (end 123.825 85.725) (width 0.25) (layer B.Cu) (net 47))
 (segment (start 141.605 111.366002) (end 147.955 117.716002) (width 1) (layer F.Cu) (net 35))
 (segment (start 147.955 117.716002) (end 147.955 120.015) (width 1) (layer F.Cu) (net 35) (status 20))
 (segment (start 141.605 109.22) (end 141.605 111.366002) (width 1) (layer F.Cu) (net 35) (status 10)))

